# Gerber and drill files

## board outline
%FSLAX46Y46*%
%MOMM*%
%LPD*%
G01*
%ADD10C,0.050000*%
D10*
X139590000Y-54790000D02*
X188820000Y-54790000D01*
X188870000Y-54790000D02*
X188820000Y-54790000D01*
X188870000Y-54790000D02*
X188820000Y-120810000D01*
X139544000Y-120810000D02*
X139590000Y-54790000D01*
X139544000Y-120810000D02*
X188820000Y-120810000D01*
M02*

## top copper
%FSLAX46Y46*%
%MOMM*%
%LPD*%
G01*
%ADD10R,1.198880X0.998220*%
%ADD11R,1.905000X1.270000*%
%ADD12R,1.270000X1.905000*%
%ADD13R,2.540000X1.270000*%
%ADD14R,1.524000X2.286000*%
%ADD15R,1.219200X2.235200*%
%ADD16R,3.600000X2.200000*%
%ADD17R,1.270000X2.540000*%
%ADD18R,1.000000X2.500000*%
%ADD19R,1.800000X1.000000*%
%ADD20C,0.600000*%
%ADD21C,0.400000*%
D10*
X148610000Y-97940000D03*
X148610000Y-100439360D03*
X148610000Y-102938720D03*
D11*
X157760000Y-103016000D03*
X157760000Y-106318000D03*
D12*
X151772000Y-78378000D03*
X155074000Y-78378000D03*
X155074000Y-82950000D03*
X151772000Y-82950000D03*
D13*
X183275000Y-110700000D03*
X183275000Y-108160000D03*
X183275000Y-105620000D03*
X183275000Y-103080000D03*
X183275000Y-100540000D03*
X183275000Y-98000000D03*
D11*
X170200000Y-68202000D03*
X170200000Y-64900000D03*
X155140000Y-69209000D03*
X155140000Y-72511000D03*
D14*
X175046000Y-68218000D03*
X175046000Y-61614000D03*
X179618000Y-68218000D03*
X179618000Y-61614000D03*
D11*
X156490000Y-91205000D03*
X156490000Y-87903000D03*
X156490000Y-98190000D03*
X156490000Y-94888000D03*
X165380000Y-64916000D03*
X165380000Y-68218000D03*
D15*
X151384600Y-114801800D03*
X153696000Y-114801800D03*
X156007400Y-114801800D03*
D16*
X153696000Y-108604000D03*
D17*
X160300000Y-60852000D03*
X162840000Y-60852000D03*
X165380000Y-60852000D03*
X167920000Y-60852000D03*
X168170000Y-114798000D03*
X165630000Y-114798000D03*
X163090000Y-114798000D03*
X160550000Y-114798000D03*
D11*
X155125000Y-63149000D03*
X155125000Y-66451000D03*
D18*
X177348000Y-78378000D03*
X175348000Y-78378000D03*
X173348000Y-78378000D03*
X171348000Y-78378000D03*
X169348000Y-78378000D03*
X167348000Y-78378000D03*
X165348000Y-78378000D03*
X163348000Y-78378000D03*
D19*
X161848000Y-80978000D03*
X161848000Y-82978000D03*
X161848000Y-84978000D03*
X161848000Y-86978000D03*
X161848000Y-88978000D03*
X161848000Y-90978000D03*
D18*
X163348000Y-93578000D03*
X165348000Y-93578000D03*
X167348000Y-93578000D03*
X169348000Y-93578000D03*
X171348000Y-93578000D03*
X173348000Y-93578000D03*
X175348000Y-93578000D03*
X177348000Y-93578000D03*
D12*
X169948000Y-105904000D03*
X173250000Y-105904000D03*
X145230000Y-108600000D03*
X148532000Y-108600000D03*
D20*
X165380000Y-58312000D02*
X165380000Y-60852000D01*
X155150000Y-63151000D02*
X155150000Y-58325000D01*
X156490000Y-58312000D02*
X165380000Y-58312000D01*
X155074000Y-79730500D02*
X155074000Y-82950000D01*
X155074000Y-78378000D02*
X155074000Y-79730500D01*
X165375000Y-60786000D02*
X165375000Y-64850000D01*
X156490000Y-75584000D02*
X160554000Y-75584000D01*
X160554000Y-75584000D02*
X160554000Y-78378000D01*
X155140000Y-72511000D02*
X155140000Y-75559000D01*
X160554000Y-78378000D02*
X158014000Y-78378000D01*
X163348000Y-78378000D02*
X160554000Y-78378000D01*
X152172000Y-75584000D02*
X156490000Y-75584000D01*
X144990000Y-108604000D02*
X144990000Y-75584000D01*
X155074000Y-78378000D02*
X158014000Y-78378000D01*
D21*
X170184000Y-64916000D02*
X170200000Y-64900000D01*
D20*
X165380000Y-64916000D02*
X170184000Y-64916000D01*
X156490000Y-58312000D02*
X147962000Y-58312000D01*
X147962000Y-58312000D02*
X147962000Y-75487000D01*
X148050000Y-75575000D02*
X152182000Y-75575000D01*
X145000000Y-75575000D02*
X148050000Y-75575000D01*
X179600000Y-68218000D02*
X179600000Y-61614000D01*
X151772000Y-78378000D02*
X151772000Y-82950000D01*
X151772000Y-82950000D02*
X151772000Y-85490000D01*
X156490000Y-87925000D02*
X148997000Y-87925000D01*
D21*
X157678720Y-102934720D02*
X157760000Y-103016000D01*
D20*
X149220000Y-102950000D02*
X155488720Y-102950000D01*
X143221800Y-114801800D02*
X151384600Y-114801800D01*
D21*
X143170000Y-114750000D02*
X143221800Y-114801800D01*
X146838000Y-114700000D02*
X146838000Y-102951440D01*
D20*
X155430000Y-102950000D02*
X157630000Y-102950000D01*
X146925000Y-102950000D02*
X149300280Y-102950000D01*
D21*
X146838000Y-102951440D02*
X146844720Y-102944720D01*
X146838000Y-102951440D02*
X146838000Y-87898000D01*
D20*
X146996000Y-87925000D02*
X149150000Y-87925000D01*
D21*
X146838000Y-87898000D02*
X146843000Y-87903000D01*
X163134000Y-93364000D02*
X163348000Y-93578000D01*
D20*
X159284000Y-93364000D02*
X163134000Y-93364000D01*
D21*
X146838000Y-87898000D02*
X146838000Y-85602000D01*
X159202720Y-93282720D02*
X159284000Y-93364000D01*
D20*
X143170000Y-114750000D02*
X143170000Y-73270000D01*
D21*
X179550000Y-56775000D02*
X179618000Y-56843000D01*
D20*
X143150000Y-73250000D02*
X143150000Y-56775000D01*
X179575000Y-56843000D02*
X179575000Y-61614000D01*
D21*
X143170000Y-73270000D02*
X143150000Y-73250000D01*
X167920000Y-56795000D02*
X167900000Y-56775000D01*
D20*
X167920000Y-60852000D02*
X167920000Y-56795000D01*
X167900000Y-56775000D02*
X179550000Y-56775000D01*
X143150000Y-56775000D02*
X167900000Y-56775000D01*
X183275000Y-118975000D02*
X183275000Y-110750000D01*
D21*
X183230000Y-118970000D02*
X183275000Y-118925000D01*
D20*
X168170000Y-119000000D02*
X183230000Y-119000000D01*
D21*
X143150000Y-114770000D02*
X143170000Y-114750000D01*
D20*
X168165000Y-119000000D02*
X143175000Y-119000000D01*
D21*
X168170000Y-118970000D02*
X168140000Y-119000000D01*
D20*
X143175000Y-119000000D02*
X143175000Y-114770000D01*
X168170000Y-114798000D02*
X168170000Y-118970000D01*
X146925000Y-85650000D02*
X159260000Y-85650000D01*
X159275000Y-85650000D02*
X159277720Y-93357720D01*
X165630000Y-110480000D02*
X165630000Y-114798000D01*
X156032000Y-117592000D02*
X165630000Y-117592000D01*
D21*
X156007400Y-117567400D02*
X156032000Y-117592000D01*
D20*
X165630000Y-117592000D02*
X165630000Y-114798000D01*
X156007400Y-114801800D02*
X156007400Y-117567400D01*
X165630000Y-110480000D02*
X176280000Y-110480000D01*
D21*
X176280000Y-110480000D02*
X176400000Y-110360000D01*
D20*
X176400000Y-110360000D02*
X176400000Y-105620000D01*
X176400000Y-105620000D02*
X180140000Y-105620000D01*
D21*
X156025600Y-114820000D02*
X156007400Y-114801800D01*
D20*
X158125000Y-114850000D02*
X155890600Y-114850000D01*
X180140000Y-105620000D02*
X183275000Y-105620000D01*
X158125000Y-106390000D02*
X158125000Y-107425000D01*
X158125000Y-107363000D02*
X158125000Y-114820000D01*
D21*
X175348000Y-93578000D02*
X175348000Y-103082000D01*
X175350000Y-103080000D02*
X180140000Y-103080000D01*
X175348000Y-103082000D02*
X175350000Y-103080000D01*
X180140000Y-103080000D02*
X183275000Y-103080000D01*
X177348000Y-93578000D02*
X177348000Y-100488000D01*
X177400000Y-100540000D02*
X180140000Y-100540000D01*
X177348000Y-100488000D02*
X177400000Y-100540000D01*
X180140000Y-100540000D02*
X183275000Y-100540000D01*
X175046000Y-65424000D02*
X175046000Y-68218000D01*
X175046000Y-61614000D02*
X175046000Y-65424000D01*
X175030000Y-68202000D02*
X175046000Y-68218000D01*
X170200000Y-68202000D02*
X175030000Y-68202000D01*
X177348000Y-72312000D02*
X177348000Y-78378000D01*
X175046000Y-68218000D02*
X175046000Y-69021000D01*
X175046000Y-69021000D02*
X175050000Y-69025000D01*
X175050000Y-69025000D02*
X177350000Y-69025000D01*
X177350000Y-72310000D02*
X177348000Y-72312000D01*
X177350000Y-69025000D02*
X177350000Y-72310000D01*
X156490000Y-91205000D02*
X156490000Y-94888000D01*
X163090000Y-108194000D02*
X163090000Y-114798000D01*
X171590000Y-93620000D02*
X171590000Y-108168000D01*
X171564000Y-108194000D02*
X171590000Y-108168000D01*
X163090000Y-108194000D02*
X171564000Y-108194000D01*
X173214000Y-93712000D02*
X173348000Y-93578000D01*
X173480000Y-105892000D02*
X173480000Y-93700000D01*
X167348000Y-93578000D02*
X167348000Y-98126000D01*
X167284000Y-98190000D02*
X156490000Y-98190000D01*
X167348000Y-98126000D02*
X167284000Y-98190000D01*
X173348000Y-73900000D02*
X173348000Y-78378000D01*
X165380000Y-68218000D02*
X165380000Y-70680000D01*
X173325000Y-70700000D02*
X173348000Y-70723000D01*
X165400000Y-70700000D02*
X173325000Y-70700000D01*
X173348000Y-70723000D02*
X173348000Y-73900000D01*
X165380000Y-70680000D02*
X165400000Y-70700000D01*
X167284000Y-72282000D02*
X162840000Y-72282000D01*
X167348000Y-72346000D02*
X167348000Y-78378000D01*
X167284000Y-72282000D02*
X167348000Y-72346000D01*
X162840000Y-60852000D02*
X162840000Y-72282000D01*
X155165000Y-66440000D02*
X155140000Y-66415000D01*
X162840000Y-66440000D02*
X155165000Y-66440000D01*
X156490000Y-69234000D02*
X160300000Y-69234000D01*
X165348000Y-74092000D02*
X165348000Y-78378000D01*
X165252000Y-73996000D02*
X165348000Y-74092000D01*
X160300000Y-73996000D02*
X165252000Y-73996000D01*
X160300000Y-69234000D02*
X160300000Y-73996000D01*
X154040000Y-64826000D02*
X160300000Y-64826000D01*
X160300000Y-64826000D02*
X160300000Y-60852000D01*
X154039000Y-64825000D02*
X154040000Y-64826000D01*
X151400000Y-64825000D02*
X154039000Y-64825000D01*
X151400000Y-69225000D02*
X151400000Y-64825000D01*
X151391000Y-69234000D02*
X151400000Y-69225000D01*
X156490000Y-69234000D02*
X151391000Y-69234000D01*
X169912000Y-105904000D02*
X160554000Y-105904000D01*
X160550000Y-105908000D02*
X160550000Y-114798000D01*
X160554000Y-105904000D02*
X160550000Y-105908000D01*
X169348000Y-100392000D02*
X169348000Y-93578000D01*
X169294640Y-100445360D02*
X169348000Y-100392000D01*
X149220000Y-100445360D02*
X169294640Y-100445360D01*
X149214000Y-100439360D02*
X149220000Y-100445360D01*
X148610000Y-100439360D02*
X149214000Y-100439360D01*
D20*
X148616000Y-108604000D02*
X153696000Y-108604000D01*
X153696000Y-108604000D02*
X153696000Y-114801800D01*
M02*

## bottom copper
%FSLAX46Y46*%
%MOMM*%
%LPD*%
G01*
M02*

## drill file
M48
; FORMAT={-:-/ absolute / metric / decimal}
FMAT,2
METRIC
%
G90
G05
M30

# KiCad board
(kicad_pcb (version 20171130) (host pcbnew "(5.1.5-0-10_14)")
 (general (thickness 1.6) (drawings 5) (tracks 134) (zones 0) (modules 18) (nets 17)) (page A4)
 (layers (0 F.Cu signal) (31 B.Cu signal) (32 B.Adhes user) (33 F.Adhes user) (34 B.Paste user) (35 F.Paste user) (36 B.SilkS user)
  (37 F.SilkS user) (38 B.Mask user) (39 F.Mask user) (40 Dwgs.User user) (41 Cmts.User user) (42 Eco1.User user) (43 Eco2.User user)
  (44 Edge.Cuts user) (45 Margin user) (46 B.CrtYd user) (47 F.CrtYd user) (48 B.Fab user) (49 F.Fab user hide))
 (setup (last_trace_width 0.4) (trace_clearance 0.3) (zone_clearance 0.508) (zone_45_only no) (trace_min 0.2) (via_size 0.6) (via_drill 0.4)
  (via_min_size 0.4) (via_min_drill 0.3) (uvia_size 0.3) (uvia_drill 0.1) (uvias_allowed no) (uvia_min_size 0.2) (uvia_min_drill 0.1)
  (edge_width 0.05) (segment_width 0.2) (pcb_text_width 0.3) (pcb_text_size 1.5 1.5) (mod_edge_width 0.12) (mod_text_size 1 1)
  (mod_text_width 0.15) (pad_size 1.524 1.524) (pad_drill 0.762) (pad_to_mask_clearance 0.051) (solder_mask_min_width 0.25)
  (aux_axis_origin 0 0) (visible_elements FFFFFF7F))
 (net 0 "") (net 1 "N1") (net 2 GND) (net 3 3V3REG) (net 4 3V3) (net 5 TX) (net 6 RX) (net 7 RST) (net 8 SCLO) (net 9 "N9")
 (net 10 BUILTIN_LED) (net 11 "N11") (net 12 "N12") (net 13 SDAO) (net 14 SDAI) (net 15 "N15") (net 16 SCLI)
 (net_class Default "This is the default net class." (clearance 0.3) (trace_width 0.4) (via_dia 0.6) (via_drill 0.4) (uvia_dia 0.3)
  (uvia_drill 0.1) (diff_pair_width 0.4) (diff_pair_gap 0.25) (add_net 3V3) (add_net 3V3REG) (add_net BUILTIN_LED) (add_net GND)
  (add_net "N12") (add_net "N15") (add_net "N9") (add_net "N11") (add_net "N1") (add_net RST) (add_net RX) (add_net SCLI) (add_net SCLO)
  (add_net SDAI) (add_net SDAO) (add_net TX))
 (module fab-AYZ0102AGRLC (layer F.Cu) (at 146.3113 100.43936 90)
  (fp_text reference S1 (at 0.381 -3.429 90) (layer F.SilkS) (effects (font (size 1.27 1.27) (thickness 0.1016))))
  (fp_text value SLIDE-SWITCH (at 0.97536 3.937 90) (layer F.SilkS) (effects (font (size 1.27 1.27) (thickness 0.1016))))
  (pad 1 smd rect (at 2.49936 2.2987 90) (size 0.99822 1.19888) (layers F.Cu F.Paste F.Mask))
  (pad 2 smd rect (at 0 2.2987 90) (size 0.99822 1.19888) (layers F.Cu F.Paste F.Mask) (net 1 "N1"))
  (pad 3 smd rect (at -2.49936 2.2987 90) (size 0.99822 1.19888) (layers F.Cu F.Paste F.Mask) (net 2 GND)))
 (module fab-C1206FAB (layer F.Cu) (at 157.76 104.667 90)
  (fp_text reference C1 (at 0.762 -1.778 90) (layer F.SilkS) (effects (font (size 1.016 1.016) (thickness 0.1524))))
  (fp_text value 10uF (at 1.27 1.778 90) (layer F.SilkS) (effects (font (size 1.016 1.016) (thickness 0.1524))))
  (pad 2 smd rect (at 1.651 0 90) (size 1.27 1.905) (layers F.Cu F.Paste F.Mask) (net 2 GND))
  (pad 1 smd rect (at -1.651 0 90) (size 1.27 1.905) (layers F.Cu F.Paste F.Mask) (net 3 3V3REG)))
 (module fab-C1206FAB (layer F.Cu) (at 153.423 78.378 180)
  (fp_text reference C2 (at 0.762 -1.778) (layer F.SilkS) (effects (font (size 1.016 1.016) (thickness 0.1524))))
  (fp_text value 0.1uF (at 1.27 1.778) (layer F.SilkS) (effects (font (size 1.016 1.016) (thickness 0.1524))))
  (pad 2 smd rect (at 1.651 0 180) (size 1.27 1.905) (layers F.Cu F.Paste F.Mask) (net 2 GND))
  (pad 1 smd rect (at -1.651 0 180) (size 1.27 1.905) (layers F.Cu F.Paste F.Mask) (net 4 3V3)))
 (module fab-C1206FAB (layer F.Cu) (at 153.423 82.95 180)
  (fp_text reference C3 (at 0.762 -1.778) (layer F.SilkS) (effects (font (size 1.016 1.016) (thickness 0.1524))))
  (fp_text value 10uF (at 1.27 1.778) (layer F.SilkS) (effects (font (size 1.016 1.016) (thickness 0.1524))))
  (pad 1 smd rect (at -1.651 0 180) (size 1.27 1.905) (layers F.Cu F.Paste F.Mask) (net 4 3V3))
  (pad 2 smd rect (at 1.651 0 180) (size 1.27 1.905) (layers F.Cu F.Paste F.Mask) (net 2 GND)))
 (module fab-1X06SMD (layer F.Cu) (at 183.275 104.35 180)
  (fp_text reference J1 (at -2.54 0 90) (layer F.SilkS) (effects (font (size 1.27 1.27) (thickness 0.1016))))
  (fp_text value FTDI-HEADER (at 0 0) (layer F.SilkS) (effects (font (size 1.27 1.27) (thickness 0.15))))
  (pad 1 smd rect (at 0 -6.35 180) (size 2.54 1.27) (layers F.Cu F.Paste F.Mask) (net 2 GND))
  (pad 2 smd rect (at 0 -3.81 180) (size 2.54 1.27) (layers F.Cu F.Paste F.Mask))
  (pad 3 smd rect (at 0 -1.27 180) (size 2.54 1.27) (layers F.Cu F.Paste F.Mask) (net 3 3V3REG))
  (pad 4 smd rect (at 0 1.27 180) (size 2.54 1.27) (layers F.Cu F.Paste F.Mask) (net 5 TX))
  (pad 5 smd rect (at 0 3.81 180) (size 2.54 1.27) (layers F.Cu F.Paste F.Mask) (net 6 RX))
  (pad 6 smd rect (at 0 6.35 180) (size 2.54 1.27) (layers F.Cu F.Paste F.Mask)))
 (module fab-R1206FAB (layer F.Cu) (at 170.2 66.551 90)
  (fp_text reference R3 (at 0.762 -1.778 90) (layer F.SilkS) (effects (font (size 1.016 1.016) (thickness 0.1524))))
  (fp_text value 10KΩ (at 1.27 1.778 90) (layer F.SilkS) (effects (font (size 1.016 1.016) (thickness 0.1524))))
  (pad 1 smd rect (at -1.651 0 90) (size 1.27 1.905) (layers F.Cu F.Paste F.Mask) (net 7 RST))
  (pad 2 smd rect (at 1.651 0 90) (size 1.27 1.905) (layers F.Cu F.Paste F.Mask) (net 4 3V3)))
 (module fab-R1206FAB (layer F.Cu) (at 155.14 70.86 270)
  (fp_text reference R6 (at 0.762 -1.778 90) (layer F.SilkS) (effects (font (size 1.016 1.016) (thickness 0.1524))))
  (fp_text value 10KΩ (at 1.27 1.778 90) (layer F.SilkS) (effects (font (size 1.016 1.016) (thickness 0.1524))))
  (pad 1 smd rect (at -1.651 0 270) (size 1.27 1.905) (layers F.Cu F.Paste F.Mask) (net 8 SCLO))
  (pad 2 smd rect (at 1.651 0 270) (size 1.27 1.905) (layers F.Cu F.Paste F.Mask) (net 4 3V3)))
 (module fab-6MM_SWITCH (layer F.Cu) (at 177.332 64.916 90)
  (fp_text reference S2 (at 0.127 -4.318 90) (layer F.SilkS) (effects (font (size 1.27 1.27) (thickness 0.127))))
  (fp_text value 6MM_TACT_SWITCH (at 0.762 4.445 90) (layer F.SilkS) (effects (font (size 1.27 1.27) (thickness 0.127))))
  (pad 1 smd rect (at -3.302 -2.286 90) (size 2.286 1.524) (layers F.Cu F.Paste F.Mask) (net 7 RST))
  (pad 2 smd rect (at 3.302 -2.286 90) (size 2.286 1.524) (layers F.Cu F.Paste F.Mask) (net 7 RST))
  (pad 3 smd rect (at -3.302 2.286 90) (size 2.286 1.524) (layers F.Cu F.Paste F.Mask) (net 2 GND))
  (pad 4 smd rect (at 3.302 2.286 90) (size 2.286 1.524) (layers F.Cu F.Paste F.Mask) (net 2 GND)))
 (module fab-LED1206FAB (layer F.Cu) (at 156.49 89.554 90)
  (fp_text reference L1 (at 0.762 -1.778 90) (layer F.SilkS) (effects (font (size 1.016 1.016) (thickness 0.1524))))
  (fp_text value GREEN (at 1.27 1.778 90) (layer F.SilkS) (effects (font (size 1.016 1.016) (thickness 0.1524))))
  (pad 1 smd rect (at -1.651 0 90) (size 1.27 1.905) (layers F.Cu F.Paste F.Mask) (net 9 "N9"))
  (pad 2 smd rect (at 1.651 0 90) (size 1.27 1.905) (layers F.Cu F.Paste F.Mask) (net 2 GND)))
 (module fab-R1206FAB (layer F.Cu) (at 156.49 96.539 90)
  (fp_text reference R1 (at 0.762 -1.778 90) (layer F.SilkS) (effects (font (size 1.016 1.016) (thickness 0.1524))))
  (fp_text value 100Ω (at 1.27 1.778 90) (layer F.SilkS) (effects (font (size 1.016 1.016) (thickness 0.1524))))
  (pad 1 smd rect (at -1.651 0 90) (size 1.27 1.905) (layers F.Cu F.Paste F.Mask) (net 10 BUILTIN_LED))
  (pad 2 smd rect (at 1.651 0 90) (size 1.27 1.905) (layers F.Cu F.Paste F.Mask) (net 9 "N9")))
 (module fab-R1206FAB (layer F.Cu) (at 165.38 66.567 90)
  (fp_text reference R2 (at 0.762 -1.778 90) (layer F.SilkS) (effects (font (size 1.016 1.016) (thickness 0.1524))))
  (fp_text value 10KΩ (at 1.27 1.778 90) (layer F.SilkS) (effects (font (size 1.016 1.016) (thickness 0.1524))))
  (pad 2 smd rect (at 1.651 0 90) (size 1.27 1.905) (layers F.Cu F.Paste F.Mask) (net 4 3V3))
  (pad 1 smd rect (at -1.651 0 90) (size 1.27 1.905) (layers F.Cu F.Paste F.Mask) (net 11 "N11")))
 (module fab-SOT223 (layer F.Cu) (at 153.696 111.703)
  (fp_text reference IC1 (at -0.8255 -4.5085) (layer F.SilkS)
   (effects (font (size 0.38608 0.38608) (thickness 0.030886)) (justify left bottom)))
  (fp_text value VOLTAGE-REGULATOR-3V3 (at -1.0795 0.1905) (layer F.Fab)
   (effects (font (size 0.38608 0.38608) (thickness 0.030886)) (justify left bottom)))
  (pad 1 smd rect (at -2.3114 3.0988) (size 1.2192 2.2352) (layers F.Cu F.Paste F.Mask) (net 2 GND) (solder_mask_margin 0.1016))
  (pad 2 smd rect (at 0 3.0988) (size 1.2192 2.2352) (layers F.Cu F.Paste F.Mask) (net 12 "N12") (solder_mask_margin 0.1016))
  (pad 3 smd rect (at 2.3114 3.0988) (size 1.2192 2.2352) (layers F.Cu F.Paste F.Mask) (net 3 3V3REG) (solder_mask_margin 0.1016))
  (pad 2 smd rect (at 0 -3.099) (size 3.6 2.2) (layers F.Cu F.Paste F.Mask) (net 12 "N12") (solder_mask_margin 0.1016)))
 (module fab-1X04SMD (layer F.Cu) (at 164.11 60.852 90)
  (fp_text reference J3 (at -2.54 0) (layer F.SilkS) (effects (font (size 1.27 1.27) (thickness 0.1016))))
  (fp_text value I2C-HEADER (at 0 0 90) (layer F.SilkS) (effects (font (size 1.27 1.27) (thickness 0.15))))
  (pad 1 smd rect (at 0 -3.81 90) (size 2.54 1.27) (layers F.Cu F.Paste F.Mask) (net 8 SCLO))
  (pad 2 smd rect (at 0 -1.27 90) (size 2.54 1.27) (layers F.Cu F.Paste F.Mask) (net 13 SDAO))
  (pad 3 smd rect (at 0 1.27 90) (size 2.54 1.27) (layers F.Cu F.Paste F.Mask) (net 4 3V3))
  (pad 4 smd rect (at 0 3.81 90) (size 2.54 1.27) (layers F.Cu F.Paste F.Mask) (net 2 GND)))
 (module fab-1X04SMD (layer F.Cu) (at 164.36 114.798 270)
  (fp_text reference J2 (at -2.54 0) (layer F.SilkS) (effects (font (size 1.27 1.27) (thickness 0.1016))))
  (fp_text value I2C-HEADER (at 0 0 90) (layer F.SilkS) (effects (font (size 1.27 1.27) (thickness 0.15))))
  (pad 1 smd rect (at 0 -3.81 270) (size 2.54 1.27) (layers F.Cu F.Paste F.Mask) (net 2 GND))
  (pad 2 smd rect (at 0 -1.27 270) (size 2.54 1.27) (layers F.Cu F.Paste F.Mask) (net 3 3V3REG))
  (pad 3 smd rect (at 0 1.27 270) (size 2.54 1.27) (layers F.Cu F.Paste F.Mask) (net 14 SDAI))
  (pad 4 smd rect (at 0 3.81 270) (size 2.54 1.27) (layers F.Cu F.Paste F.Mask) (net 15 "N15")))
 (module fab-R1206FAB (layer F.Cu) (at 155.125 64.8 90)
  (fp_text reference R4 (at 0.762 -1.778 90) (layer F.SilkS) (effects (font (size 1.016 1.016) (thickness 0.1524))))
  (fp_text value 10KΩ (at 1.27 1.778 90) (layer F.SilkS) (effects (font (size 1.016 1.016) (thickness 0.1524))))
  (pad 2 smd rect (at 1.651 0 90) (size 1.27 1.905) (layers F.Cu F.Paste F.Mask) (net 4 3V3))
  (pad 1 smd rect (at -1.651 0 90) (size 1.27 1.905) (layers F.Cu F.Paste F.Mask) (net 13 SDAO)))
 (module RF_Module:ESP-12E (layer F.Cu) (at 173.848 85.978 270)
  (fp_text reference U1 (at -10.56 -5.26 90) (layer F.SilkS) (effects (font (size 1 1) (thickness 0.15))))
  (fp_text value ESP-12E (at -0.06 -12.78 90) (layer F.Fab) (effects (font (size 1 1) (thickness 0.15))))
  (pad 1 smd rect (at -7.6 -3.5 270) (size 2.5 1) (layers F.Cu F.Paste F.Mask) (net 7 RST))
  (pad 2 smd rect (at -7.6 -1.5 270) (size 2.5 1) (layers F.Cu F.Paste F.Mask))
  (pad 3 smd rect (at -7.6 0.5 270) (size 2.5 1) (layers F.Cu F.Paste F.Mask) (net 11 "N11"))
  (pad 4 smd rect (at -7.6 2.5 270) (size 2.5 1) (layers F.Cu F.Paste F.Mask))
  (pad 5 smd rect (at -7.6 4.5 270) (size 2.5 1) (layers F.Cu F.Paste F.Mask))
  (pad 6 smd rect (at -7.6 6.5 270) (size 2.5 1) (layers F.Cu F.Paste F.Mask) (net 13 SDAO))
  (pad 7 smd rect (at -7.6 8.5 270) (size 2.5 1) (layers F.Cu F.Paste F.Mask) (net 8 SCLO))
  (pad 8 smd rect (at -7.6 10.5 270) (size 2.5 1) (layers F.Cu F.Paste F.Mask) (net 4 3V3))
  (pad 9 smd rect (at -5 12 270) (size 1 1.8) (layers F.Cu F.Paste F.Mask))
  (pad 10 smd rect (at -3 12 270) (size 1 1.8) (layers F.Cu F.Paste F.Mask))
  (pad 11 smd rect (at -1 12 270) (size 1 1.8) (layers F.Cu F.Paste F.Mask))
  (pad 12 smd rect (at 1 12 270) (size 1 1.8) (layers F.Cu F.Paste F.Mask))
  (pad 13 smd rect (at 3 12 270) (size 1 1.8) (layers F.Cu F.Paste F.Mask))
  (pad 14 smd rect (at 5 12 270) (size 1 1.8) (layers F.Cu F.Paste F.Mask))
  (pad 15 smd rect (at 7.6 10.5 270) (size 2.5 1) (layers F.Cu F.Paste F.Mask) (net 2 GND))
  (pad 16 smd rect (at 7.6 8.5 270) (size 2.5 1) (layers F.Cu F.Paste F.Mask))
  (pad 17 smd rect (at 7.6 6.5 270) (size 2.5 1) (layers F.Cu F.Paste F.Mask) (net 10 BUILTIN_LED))
  (pad 18 smd rect (at 7.6 4.5 270) (size 2.5 1) (layers F.Cu F.Paste F.Mask) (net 1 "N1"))
  (pad 19 smd rect (at 7.6 2.5 270) (size 2.5 1) (layers F.Cu F.Paste F.Mask) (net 14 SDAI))
  (pad 20 smd rect (at 7.6 0.5 270) (size 2.5 1) (layers F.Cu F.Paste F.Mask) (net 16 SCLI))
  (pad 21 smd rect (at 7.6 -1.5 270) (size 2.5 1) (layers F.Cu F.Paste F.Mask) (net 5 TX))
  (pad 22 smd rect (at 7.6 -3.5 270) (size 2.5 1) (layers F.Cu F.Paste F.Mask) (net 6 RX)))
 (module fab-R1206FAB (layer F.Cu) (at 171.599 105.904)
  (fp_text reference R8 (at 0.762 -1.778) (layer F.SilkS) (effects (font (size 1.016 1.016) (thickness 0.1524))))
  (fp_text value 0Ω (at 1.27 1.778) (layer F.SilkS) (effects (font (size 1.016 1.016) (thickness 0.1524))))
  (pad 1 smd rect (at -1.651 0) (size 1.27 1.905) (layers F.Cu F.Paste F.Mask) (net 15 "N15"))
  (pad 2 smd rect (at 1.651 0) (size 1.27 1.905) (layers F.Cu F.Paste F.Mask) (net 16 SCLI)))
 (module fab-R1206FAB (layer F.Cu) (at 146.881 108.6)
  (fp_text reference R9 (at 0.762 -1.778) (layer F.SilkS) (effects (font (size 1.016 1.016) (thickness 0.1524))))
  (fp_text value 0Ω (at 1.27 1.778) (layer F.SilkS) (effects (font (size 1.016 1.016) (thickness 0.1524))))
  (pad 1 smd rect (at -1.651 0) (size 1.27 1.905) (layers F.Cu F.Paste F.Mask) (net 4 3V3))
  (pad 2 smd rect (at 1.651 0) (size 1.27 1.905) (layers F.Cu F.Paste F.Mask) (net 12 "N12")))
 (gr_line (start 139.59 54.79) (end 188.82 54.79) (layer Edge.Cuts) (width 0.05))
 (gr_line (start 188.87 54.79) (end 188.82 54.79) (layer Edge.Cuts) (width 0.05))
 (gr_line (start 188.87 54.79) (end 188.82 120.81) (layer Edge.Cuts) (width 0.05))
 (gr_line (start 139.544 120.81) (end 139.59 54.79) (layer Edge.Cuts) (width 0.05))
 (gr_line (start 139.544 120.81) (end 188.82 120.81) (layer Edge.Cuts) (width 0.05))
 (segment (start 165.38 58.312) (end 165.38 60.852) (width 0.6) (layer F.Cu) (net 4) (status 20))
 (segment (start 155.15 63.151) (end 155.15 58.325) (width 0.6) (layer F.Cu) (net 4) (status 10))
 (segment (start 156.49 58.312) (end 165.38 58.312) (width 0.6) (layer F.Cu) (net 4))
 (segment (start 155.074 79.7305) (end 155.074 82.95) (width 0.6) (layer F.Cu) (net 4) (status 20))
 (segment (start 155.074 78.378) (end 155.074 79.7305) (width 0.6) (layer F.Cu) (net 4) (status 10))
 (segment (start 165.375 60.786) (end 165.375 64.85) (width 0.6) (layer F.Cu) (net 4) (status 30))
 (segment (start 156.49 75.584) (end 160.554 75.584) (width 0.6) (layer F.Cu) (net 4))
 (segment (start 160.554 75.584) (end 160.554 78.378) (width 0.6) (layer F.Cu) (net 4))
 (segment (start 155.14 72.511) (end 155.14 75.559) (width 0.6) (layer F.Cu) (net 4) (status 10))
 (segment (start 160.554 78.378) (end 158.014 78.378) (width 0.6) (layer F.Cu) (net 4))
 (segment (start 163.348 78.378) (end 160.554 78.378) (width 0.6) (layer F.Cu) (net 4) (status 10))
 (segment (start 152.172 75.584) (end 156.49 75.584) (width 0.6) (layer F.Cu) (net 4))
 (segment (start 144.99 108.604) (end 144.99 75.584) (width 0.6) (layer F.Cu) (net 4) (status 10))
 (segment (start 155.074 78.378) (end 158.014 78.378) (width 0.6) (layer F.Cu) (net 4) (status 10))
 (segment (start 170.184 64.916) (end 170.2 64.9) (width 0.4) (layer F.Cu) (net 4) (status 30))
 (segment (start 165.38 64.916) (end 170.184 64.916) (width 0.6) (layer F.Cu) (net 4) (status 30))
 (segment (start 156.49 58.312) (end 147.962 58.312) (width 0.6) (layer F.Cu) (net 4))
 (segment (start 147.962 58.312) (end 147.962 75.487) (width 0.6) (layer F.Cu) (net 4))
 (segment (start 148.05 75.575) (end 152.182 75.575) (width 0.6) (layer F.Cu) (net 4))
 (segment (start 145 75.575) (end 148.05 75.575) (width 0.6) (layer F.Cu) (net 4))
 (segment (start 179.6 68.218) (end 179.6 61.614) (width 0.6) (layer F.Cu) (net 2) (status 30))
 (segment (start 151.772 78.378) (end 151.772 82.95) (width 0.6) (layer F.Cu) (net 2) (status 30))
 (segment (start 151.772 82.95) (end 151.772 85.49) (width 0.6) (layer F.Cu) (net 2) (status 10))
 (segment (start 156.49 87.925) (end 148.997 87.925) (width 0.6) (layer F.Cu) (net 2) (status 10))
 (segment (start 157.67872 102.93472) (end 157.76 103.016) (width 0.4) (layer F.Cu) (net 2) (status 30))
 (segment (start 149.22 102.95) (end 155.48872 102.95) (width 0.6) (layer F.Cu) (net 2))
 (segment (start 143.2218 114.8018) (end 151.3846 114.8018) (width 0.6) (layer F.Cu) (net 2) (status 20))
 (segment (start 143.17 114.75) (end 143.2218 114.8018) (width 0.4) (layer F.Cu) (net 2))
 (segment (start 146.838 114.7) (end 146.838 102.95144) (width 0.4) (layer F.Cu) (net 2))
 (segment (start 155.43 102.95) (end 157.63 102.95) (width 0.6) (layer F.Cu) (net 2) (status 20))
 (segment (start 146.925 102.95) (end 149.30028 102.95) (width 0.6) (layer F.Cu) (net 2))
 (segment (start 146.838 102.95144) (end 146.84472 102.94472) (width 0.4) (layer F.Cu) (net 2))
 (segment (start 146.838 102.95144) (end 146.838 87.898) (width 0.4) (layer F.Cu) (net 2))
 (segment (start 146.996 87.925) (end 149.15 87.925) (width 0.6) (layer F.Cu) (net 2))
 (segment (start 146.838 87.898) (end 146.843 87.903) (width 0.4) (layer F.Cu) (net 2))
 (segment (start 163.134 93.364) (end 163.348 93.578) (width 0.4) (layer F.Cu) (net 2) (status 30))
 (segment (start 159.284 93.364) (end 163.134 93.364) (width 0.6) (layer F.Cu) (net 2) (status 20))
 (segment (start 146.838 87.898) (end 146.838 85.602) (width 0.4) (layer F.Cu) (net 2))
 (segment (start 159.20272 93.28272) (end 159.284 93.364) (width 0.4) (layer F.Cu) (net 2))
 (segment (start 143.17 114.75) (end 143.17 73.27) (width 0.6) (layer F.Cu) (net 2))
 (segment (start 179.55 56.775) (end 179.618 56.843) (width 0.4) (layer F.Cu) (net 2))
 (segment (start 143.15 73.25) (end 143.15 56.775) (width 0.6) (layer F.Cu) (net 2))
 (segment (start 179.575 56.843) (end 179.575 61.614) (width 0.6) (layer F.Cu) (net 2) (status 20))
 (segment (start 143.17 73.27) (end 143.15 73.25) (width 0.4) (layer F.Cu) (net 2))
 (segment (start 167.92 56.795) (end 167.9 56.775) (width 0.4) (layer F.Cu) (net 2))
 (segment (start 167.92 60.852) (end 167.92 56.795) (width 0.6) (layer F.Cu) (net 2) (status 10))
 (segment (start 167.9 56.775) (end 179.55 56.775) (width 0.6) (layer F.Cu) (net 2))
 (segment (start 143.15 56.775) (end 167.9 56.775) (width 0.6) (layer F.Cu) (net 2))
 (segment (start 183.275 118.975) (end 183.275 110.75) (width 0.6) (layer F.Cu) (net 2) (status 20))
 (segment (start 183.23 118.97) (end 183.275 118.925) (width 0.4) (layer F.Cu) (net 2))
 (segment (start 168.17 119) (end 183.23 119) (width 0.6) (layer F.Cu) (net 2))
 (segment (start 143.15 114.77) (end 143.17 114.75) (width 0.4) (layer F.Cu) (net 2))
 (segment (start 168.165 119) (end 143.175 119) (width 0.6) (layer F.Cu) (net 2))
 (segment (start 168.17 118.97) (end 168.14 119) (width 0.4) (layer F.Cu) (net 2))
 (segment (start 143.175 119) (end 143.175 114.77) (width 0.6) (layer F.Cu) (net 2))
 (segment (start 168.17 114.798) (end 168.17 118.97) (width 0.6) (layer F.Cu) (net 2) (status 10))
 (segment (start 146.925 85.65) (end 159.26 85.65) (width 0.6) (layer F.Cu) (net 2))
 (segment (start 159.275 85.65) (end 159.27772 93.35772) (width 0.6) (layer F.Cu) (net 2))
 (segment (start 165.63 110.48) (end 165.63 114.798) (width 0.6) (layer F.Cu) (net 3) (status 20))
 (segment (start 156.032 117.592) (end 165.63 117.592) (width 0.6) (layer F.Cu) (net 3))
 (segment (start 156.0074 117.5674) (end 156.032 117.592) (width 0.4) (layer F.Cu) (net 3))
 (segment (start 165.63 117.592) (end 165.63 114.798) (width 0.6) (layer F.Cu) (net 3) (status 20))
 (segment (start 156.0074 114.8018) (end 156.0074 117.5674) (width 0.6) (layer F.Cu) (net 3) (status 10))
 (segment (start 165.63 110.48) (end 176.28 110.48) (width 0.6) (layer F.Cu) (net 3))
 (segment (start 176.28 110.48) (end 176.4 110.36) (width 0.4) (layer F.Cu) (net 3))
 (segment (start 176.4 110.36) (end 176.4 105.62) (width 0.6) (layer F.Cu) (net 3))
 (segment (start 176.4 105.62) (end 180.14 105.62) (width 0.6) (layer F.Cu) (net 3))
 (segment (start 156.0256 114.82) (end 156.0074 114.8018) (width 0.4) (layer F.Cu) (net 3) (status 30))
 (segment (start 158.125 114.85) (end 155.8906 114.85) (width 0.6) (layer F.Cu) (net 3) (status 20))
 (segment (start 180.14 105.62) (end 183.275 105.62) (width 0.6) (layer F.Cu) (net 3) (status 20))
 (segment (start 158.125 106.39) (end 158.125 107.425) (width 0.6) (layer F.Cu) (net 3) (status 10))
 (segment (start 158.125 107.363) (end 158.125 114.82) (width 0.6) (layer F.Cu) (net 3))
 (segment (start 175.348 93.578) (end 175.348 103.082) (width 0.4) (layer F.Cu) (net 5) (status 10))
 (segment (start 175.35 103.08) (end 180.14 103.08) (width 0.4) (layer F.Cu) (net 5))
 (segment (start 175.348 103.082) (end 175.35 103.08) (width 0.4) (layer F.Cu) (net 5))
 (segment (start 180.14 103.08) (end 183.275 103.08) (width 0.4) (layer F.Cu) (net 5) (status 20))
 (segment (start 177.348 93.578) (end 177.348 100.488) (width 0.4) (layer F.Cu) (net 6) (status 10))
 (segment (start 177.4 100.54) (end 180.14 100.54) (width 0.4) (layer F.Cu) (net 6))
 (segment (start 177.348 100.488) (end 177.4 100.54) (width 0.4) (layer F.Cu) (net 6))
 (segment (start 180.14 100.54) (end 183.275 100.54) (width 0.4) (layer F.Cu) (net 6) (status 20))
 (segment (start 175.046 65.424) (end 175.046 68.218) (width 0.4) (layer F.Cu) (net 7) (status 20))
 (segment (start 175.046 61.614) (end 175.046 65.424) (width 0.4) (layer F.Cu) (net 7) (status 10))
 (segment (start 175.03 68.202) (end 175.046 68.218) (width 0.4) (layer F.Cu) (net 7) (status 30))
 (segment (start 170.2 68.202) (end 175.03 68.202) (width 0.4) (layer F.Cu) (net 7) (status 30))
 (segment (start 177.348 72.312) (end 177.348 78.378) (width 0.4) (layer F.Cu) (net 7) (status 20))
 (segment (start 175.046 68.218) (end 175.046 69.021) (width 0.4) (layer F.Cu) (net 7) (status 30))
 (segment (start 175.046 69.021) (end 175.05 69.025) (width 0.4) (layer F.Cu) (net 7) (status 30))
 (segment (start 175.05 69.025) (end 177.35 69.025) (width 0.4) (layer F.Cu) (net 7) (status 10))
 (segment (start 177.35 72.31) (end 177.348 72.312) (width 0.4) (layer F.Cu) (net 7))
 (segment (start 177.35 69.025) (end 177.35 72.31) (width 0.4) (layer F.Cu) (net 7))
 (segment (start 156.49 91.205) (end 156.49 94.888) (width 0.4) (layer F.Cu) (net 9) (status 30))
 (segment (start 163.09 108.194) (end 163.09 114.798) (width 0.4) (layer F.Cu) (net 14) (status 20))
 (segment (start 171.59 93.62) (end 171.59 108.168) (width 0.4) (layer F.Cu) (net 14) (status 10))
 (segment (start 171.564 108.194) (end 171.59 108.168) (width 0.4) (layer F.Cu) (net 14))
 (segment (start 163.09 108.194) (end 171.564 108.194) (width 0.4) (layer F.Cu) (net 14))
 (segment (start 173.214 93.712) (end 173.348 93.578) (width 0.4) (layer F.Cu) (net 16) (status 30))
 (segment (start 173.48 105.892) (end 173.48 93.7) (width 0.4) (layer F.Cu) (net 16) (status 30))
 (segment (start 167.348 93.578) (end 167.348 98.126) (width 0.4) (layer F.Cu) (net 10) (status 10))
 (segment (start 167.284 98.19) (end 156.49 98.19) (width 0.4) (layer F.Cu) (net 10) (status 20))
 (segment (start 167.348 98.126) (end 167.284 98.19) (width 0.4) (layer F.Cu) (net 10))
 (segment (start 173.348 73.9) (end 173.348 78.378) (width 0.4) (layer F.Cu) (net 11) (status 20))
 (segment (start 165.38 68.218) (end 165.38 70.68) (width 0.4) (layer F.Cu) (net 11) (status 10))
 (segment (start 173.325 70.7) (end 173.348 70.723) (width 0.4) (layer F.Cu) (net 11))
 (segment (start 165.4 70.7) (end 173.325 70.7) (width 0.4) (layer F.Cu) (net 11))
 (segment (start 173.348 70.723) (end 173.348 73.9) (width 0.4) (layer F.Cu) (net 11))
 (segment (start 165.38 70.68) (end 165.4 70.7) (width 0.4) (layer F.Cu) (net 11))
 (segment (start 167.284 72.282) (end 162.84 72.282) (width 0.4) (layer F.Cu) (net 13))
 (segment (start 167.348 72.346) (end 167.348 78.378) (width 0.4) (layer F.Cu) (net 13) (status 20))
 (segment (start 167.284 72.282) (end 167.348 72.346) (width 0.4) (layer F.Cu) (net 13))
 (segment (start 162.84 60.852) (end 162.84 72.282) (width 0.4) (layer F.Cu) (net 13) (status 10))
 (segment (start 155.165 66.44) (end 155.14 66.415) (width 0.4) (layer F.Cu) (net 13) (status 30))
 (segment (start 162.84 66.44) (end 155.165 66.44) (width 0.4) (layer F.Cu) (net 13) (status 20))
 (segment (start 156.49 69.234) (end 160.3 69.234) (width 0.4) (layer F.Cu) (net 8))
 (segment (start 165.348 74.092) (end 165.348 78.378) (width 0.4) (layer F.Cu) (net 8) (status 20))
 (segment (start 165.252 73.996) (end 165.348 74.092) (width 0.4) (layer F.Cu) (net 8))
 (segment (start 160.3 73.996) (end 165.252 73.996) (width 0.4) (layer F.Cu) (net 8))
 (segment (start 160.3 69.234) (end 160.3 73.996) (width 0.4) (layer F.Cu) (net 8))
 (segment (start 154.04 64.826) (end 160.3 64.826) (width 0.4) (layer F.Cu) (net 8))
 (segment (start 160.3 64.826) (end 160.3 60.852) (width 0.4) (layer F.Cu) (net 8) (status 20))
 (segment (start 154.039 64.825) (end 154.04 64.826) (width 0.4) (layer F.Cu) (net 8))
 (segment (start 151.4 64.825) (end 154.039 64.825) (width 0.4) (layer F.Cu) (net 8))
 (segment (start 151.4 69.225) (end 151.4 64.825) (width 0.4) (layer F.Cu) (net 8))
 (segment (start 151.391 69.234) (end 151.4 69.225) (width 0.4) (layer F.Cu) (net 8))
 (segment (start 156.49 69.234) (end 151.391 69.234) (width 0.4) (layer F.Cu) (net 8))
 (segment (start 169.912 105.904) (end 160.554 105.904) (width 0.4) (layer F.Cu) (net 15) (status 10))
 (segment (start 160.55 105.908) (end 160.55 114.798) (width 0.4) (layer F.Cu) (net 15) (status 20))
 (segment (start 160.554 105.904) (end 160.55 105.908) (width 0.4) (layer F.Cu) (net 15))
 (segment (start 169.348 100.392) (end 169.348 93.578) (width 0.4) (layer F.Cu) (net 1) (status 20))
 (segment (start 169.29464 100.44536) (end 169.348 100.392) (width 0.4) (layer F.Cu) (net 1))
 (segment (start 149.22 100.44536) (end 169.29464 100.44536) (width 0.4) (layer F.Cu) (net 1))
 (segment (start 149.214 100.43936) (end 149.22 100.44536) (width 0.4) (layer F.Cu) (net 1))
 (segment (start 148.61 100.43936) (end 149.214 100.43936) (width 0.4) (layer F.Cu) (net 1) (status 10))
 (segment (start 148.616 108.604) (end 153.696 108.604) (width 0.6) (layer F.Cu) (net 12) (status 30))
 (segment (start 153.696 108.604) (end 153.696 114.8018) (width 0.6) (layer F.Cu) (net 12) (status 30)))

